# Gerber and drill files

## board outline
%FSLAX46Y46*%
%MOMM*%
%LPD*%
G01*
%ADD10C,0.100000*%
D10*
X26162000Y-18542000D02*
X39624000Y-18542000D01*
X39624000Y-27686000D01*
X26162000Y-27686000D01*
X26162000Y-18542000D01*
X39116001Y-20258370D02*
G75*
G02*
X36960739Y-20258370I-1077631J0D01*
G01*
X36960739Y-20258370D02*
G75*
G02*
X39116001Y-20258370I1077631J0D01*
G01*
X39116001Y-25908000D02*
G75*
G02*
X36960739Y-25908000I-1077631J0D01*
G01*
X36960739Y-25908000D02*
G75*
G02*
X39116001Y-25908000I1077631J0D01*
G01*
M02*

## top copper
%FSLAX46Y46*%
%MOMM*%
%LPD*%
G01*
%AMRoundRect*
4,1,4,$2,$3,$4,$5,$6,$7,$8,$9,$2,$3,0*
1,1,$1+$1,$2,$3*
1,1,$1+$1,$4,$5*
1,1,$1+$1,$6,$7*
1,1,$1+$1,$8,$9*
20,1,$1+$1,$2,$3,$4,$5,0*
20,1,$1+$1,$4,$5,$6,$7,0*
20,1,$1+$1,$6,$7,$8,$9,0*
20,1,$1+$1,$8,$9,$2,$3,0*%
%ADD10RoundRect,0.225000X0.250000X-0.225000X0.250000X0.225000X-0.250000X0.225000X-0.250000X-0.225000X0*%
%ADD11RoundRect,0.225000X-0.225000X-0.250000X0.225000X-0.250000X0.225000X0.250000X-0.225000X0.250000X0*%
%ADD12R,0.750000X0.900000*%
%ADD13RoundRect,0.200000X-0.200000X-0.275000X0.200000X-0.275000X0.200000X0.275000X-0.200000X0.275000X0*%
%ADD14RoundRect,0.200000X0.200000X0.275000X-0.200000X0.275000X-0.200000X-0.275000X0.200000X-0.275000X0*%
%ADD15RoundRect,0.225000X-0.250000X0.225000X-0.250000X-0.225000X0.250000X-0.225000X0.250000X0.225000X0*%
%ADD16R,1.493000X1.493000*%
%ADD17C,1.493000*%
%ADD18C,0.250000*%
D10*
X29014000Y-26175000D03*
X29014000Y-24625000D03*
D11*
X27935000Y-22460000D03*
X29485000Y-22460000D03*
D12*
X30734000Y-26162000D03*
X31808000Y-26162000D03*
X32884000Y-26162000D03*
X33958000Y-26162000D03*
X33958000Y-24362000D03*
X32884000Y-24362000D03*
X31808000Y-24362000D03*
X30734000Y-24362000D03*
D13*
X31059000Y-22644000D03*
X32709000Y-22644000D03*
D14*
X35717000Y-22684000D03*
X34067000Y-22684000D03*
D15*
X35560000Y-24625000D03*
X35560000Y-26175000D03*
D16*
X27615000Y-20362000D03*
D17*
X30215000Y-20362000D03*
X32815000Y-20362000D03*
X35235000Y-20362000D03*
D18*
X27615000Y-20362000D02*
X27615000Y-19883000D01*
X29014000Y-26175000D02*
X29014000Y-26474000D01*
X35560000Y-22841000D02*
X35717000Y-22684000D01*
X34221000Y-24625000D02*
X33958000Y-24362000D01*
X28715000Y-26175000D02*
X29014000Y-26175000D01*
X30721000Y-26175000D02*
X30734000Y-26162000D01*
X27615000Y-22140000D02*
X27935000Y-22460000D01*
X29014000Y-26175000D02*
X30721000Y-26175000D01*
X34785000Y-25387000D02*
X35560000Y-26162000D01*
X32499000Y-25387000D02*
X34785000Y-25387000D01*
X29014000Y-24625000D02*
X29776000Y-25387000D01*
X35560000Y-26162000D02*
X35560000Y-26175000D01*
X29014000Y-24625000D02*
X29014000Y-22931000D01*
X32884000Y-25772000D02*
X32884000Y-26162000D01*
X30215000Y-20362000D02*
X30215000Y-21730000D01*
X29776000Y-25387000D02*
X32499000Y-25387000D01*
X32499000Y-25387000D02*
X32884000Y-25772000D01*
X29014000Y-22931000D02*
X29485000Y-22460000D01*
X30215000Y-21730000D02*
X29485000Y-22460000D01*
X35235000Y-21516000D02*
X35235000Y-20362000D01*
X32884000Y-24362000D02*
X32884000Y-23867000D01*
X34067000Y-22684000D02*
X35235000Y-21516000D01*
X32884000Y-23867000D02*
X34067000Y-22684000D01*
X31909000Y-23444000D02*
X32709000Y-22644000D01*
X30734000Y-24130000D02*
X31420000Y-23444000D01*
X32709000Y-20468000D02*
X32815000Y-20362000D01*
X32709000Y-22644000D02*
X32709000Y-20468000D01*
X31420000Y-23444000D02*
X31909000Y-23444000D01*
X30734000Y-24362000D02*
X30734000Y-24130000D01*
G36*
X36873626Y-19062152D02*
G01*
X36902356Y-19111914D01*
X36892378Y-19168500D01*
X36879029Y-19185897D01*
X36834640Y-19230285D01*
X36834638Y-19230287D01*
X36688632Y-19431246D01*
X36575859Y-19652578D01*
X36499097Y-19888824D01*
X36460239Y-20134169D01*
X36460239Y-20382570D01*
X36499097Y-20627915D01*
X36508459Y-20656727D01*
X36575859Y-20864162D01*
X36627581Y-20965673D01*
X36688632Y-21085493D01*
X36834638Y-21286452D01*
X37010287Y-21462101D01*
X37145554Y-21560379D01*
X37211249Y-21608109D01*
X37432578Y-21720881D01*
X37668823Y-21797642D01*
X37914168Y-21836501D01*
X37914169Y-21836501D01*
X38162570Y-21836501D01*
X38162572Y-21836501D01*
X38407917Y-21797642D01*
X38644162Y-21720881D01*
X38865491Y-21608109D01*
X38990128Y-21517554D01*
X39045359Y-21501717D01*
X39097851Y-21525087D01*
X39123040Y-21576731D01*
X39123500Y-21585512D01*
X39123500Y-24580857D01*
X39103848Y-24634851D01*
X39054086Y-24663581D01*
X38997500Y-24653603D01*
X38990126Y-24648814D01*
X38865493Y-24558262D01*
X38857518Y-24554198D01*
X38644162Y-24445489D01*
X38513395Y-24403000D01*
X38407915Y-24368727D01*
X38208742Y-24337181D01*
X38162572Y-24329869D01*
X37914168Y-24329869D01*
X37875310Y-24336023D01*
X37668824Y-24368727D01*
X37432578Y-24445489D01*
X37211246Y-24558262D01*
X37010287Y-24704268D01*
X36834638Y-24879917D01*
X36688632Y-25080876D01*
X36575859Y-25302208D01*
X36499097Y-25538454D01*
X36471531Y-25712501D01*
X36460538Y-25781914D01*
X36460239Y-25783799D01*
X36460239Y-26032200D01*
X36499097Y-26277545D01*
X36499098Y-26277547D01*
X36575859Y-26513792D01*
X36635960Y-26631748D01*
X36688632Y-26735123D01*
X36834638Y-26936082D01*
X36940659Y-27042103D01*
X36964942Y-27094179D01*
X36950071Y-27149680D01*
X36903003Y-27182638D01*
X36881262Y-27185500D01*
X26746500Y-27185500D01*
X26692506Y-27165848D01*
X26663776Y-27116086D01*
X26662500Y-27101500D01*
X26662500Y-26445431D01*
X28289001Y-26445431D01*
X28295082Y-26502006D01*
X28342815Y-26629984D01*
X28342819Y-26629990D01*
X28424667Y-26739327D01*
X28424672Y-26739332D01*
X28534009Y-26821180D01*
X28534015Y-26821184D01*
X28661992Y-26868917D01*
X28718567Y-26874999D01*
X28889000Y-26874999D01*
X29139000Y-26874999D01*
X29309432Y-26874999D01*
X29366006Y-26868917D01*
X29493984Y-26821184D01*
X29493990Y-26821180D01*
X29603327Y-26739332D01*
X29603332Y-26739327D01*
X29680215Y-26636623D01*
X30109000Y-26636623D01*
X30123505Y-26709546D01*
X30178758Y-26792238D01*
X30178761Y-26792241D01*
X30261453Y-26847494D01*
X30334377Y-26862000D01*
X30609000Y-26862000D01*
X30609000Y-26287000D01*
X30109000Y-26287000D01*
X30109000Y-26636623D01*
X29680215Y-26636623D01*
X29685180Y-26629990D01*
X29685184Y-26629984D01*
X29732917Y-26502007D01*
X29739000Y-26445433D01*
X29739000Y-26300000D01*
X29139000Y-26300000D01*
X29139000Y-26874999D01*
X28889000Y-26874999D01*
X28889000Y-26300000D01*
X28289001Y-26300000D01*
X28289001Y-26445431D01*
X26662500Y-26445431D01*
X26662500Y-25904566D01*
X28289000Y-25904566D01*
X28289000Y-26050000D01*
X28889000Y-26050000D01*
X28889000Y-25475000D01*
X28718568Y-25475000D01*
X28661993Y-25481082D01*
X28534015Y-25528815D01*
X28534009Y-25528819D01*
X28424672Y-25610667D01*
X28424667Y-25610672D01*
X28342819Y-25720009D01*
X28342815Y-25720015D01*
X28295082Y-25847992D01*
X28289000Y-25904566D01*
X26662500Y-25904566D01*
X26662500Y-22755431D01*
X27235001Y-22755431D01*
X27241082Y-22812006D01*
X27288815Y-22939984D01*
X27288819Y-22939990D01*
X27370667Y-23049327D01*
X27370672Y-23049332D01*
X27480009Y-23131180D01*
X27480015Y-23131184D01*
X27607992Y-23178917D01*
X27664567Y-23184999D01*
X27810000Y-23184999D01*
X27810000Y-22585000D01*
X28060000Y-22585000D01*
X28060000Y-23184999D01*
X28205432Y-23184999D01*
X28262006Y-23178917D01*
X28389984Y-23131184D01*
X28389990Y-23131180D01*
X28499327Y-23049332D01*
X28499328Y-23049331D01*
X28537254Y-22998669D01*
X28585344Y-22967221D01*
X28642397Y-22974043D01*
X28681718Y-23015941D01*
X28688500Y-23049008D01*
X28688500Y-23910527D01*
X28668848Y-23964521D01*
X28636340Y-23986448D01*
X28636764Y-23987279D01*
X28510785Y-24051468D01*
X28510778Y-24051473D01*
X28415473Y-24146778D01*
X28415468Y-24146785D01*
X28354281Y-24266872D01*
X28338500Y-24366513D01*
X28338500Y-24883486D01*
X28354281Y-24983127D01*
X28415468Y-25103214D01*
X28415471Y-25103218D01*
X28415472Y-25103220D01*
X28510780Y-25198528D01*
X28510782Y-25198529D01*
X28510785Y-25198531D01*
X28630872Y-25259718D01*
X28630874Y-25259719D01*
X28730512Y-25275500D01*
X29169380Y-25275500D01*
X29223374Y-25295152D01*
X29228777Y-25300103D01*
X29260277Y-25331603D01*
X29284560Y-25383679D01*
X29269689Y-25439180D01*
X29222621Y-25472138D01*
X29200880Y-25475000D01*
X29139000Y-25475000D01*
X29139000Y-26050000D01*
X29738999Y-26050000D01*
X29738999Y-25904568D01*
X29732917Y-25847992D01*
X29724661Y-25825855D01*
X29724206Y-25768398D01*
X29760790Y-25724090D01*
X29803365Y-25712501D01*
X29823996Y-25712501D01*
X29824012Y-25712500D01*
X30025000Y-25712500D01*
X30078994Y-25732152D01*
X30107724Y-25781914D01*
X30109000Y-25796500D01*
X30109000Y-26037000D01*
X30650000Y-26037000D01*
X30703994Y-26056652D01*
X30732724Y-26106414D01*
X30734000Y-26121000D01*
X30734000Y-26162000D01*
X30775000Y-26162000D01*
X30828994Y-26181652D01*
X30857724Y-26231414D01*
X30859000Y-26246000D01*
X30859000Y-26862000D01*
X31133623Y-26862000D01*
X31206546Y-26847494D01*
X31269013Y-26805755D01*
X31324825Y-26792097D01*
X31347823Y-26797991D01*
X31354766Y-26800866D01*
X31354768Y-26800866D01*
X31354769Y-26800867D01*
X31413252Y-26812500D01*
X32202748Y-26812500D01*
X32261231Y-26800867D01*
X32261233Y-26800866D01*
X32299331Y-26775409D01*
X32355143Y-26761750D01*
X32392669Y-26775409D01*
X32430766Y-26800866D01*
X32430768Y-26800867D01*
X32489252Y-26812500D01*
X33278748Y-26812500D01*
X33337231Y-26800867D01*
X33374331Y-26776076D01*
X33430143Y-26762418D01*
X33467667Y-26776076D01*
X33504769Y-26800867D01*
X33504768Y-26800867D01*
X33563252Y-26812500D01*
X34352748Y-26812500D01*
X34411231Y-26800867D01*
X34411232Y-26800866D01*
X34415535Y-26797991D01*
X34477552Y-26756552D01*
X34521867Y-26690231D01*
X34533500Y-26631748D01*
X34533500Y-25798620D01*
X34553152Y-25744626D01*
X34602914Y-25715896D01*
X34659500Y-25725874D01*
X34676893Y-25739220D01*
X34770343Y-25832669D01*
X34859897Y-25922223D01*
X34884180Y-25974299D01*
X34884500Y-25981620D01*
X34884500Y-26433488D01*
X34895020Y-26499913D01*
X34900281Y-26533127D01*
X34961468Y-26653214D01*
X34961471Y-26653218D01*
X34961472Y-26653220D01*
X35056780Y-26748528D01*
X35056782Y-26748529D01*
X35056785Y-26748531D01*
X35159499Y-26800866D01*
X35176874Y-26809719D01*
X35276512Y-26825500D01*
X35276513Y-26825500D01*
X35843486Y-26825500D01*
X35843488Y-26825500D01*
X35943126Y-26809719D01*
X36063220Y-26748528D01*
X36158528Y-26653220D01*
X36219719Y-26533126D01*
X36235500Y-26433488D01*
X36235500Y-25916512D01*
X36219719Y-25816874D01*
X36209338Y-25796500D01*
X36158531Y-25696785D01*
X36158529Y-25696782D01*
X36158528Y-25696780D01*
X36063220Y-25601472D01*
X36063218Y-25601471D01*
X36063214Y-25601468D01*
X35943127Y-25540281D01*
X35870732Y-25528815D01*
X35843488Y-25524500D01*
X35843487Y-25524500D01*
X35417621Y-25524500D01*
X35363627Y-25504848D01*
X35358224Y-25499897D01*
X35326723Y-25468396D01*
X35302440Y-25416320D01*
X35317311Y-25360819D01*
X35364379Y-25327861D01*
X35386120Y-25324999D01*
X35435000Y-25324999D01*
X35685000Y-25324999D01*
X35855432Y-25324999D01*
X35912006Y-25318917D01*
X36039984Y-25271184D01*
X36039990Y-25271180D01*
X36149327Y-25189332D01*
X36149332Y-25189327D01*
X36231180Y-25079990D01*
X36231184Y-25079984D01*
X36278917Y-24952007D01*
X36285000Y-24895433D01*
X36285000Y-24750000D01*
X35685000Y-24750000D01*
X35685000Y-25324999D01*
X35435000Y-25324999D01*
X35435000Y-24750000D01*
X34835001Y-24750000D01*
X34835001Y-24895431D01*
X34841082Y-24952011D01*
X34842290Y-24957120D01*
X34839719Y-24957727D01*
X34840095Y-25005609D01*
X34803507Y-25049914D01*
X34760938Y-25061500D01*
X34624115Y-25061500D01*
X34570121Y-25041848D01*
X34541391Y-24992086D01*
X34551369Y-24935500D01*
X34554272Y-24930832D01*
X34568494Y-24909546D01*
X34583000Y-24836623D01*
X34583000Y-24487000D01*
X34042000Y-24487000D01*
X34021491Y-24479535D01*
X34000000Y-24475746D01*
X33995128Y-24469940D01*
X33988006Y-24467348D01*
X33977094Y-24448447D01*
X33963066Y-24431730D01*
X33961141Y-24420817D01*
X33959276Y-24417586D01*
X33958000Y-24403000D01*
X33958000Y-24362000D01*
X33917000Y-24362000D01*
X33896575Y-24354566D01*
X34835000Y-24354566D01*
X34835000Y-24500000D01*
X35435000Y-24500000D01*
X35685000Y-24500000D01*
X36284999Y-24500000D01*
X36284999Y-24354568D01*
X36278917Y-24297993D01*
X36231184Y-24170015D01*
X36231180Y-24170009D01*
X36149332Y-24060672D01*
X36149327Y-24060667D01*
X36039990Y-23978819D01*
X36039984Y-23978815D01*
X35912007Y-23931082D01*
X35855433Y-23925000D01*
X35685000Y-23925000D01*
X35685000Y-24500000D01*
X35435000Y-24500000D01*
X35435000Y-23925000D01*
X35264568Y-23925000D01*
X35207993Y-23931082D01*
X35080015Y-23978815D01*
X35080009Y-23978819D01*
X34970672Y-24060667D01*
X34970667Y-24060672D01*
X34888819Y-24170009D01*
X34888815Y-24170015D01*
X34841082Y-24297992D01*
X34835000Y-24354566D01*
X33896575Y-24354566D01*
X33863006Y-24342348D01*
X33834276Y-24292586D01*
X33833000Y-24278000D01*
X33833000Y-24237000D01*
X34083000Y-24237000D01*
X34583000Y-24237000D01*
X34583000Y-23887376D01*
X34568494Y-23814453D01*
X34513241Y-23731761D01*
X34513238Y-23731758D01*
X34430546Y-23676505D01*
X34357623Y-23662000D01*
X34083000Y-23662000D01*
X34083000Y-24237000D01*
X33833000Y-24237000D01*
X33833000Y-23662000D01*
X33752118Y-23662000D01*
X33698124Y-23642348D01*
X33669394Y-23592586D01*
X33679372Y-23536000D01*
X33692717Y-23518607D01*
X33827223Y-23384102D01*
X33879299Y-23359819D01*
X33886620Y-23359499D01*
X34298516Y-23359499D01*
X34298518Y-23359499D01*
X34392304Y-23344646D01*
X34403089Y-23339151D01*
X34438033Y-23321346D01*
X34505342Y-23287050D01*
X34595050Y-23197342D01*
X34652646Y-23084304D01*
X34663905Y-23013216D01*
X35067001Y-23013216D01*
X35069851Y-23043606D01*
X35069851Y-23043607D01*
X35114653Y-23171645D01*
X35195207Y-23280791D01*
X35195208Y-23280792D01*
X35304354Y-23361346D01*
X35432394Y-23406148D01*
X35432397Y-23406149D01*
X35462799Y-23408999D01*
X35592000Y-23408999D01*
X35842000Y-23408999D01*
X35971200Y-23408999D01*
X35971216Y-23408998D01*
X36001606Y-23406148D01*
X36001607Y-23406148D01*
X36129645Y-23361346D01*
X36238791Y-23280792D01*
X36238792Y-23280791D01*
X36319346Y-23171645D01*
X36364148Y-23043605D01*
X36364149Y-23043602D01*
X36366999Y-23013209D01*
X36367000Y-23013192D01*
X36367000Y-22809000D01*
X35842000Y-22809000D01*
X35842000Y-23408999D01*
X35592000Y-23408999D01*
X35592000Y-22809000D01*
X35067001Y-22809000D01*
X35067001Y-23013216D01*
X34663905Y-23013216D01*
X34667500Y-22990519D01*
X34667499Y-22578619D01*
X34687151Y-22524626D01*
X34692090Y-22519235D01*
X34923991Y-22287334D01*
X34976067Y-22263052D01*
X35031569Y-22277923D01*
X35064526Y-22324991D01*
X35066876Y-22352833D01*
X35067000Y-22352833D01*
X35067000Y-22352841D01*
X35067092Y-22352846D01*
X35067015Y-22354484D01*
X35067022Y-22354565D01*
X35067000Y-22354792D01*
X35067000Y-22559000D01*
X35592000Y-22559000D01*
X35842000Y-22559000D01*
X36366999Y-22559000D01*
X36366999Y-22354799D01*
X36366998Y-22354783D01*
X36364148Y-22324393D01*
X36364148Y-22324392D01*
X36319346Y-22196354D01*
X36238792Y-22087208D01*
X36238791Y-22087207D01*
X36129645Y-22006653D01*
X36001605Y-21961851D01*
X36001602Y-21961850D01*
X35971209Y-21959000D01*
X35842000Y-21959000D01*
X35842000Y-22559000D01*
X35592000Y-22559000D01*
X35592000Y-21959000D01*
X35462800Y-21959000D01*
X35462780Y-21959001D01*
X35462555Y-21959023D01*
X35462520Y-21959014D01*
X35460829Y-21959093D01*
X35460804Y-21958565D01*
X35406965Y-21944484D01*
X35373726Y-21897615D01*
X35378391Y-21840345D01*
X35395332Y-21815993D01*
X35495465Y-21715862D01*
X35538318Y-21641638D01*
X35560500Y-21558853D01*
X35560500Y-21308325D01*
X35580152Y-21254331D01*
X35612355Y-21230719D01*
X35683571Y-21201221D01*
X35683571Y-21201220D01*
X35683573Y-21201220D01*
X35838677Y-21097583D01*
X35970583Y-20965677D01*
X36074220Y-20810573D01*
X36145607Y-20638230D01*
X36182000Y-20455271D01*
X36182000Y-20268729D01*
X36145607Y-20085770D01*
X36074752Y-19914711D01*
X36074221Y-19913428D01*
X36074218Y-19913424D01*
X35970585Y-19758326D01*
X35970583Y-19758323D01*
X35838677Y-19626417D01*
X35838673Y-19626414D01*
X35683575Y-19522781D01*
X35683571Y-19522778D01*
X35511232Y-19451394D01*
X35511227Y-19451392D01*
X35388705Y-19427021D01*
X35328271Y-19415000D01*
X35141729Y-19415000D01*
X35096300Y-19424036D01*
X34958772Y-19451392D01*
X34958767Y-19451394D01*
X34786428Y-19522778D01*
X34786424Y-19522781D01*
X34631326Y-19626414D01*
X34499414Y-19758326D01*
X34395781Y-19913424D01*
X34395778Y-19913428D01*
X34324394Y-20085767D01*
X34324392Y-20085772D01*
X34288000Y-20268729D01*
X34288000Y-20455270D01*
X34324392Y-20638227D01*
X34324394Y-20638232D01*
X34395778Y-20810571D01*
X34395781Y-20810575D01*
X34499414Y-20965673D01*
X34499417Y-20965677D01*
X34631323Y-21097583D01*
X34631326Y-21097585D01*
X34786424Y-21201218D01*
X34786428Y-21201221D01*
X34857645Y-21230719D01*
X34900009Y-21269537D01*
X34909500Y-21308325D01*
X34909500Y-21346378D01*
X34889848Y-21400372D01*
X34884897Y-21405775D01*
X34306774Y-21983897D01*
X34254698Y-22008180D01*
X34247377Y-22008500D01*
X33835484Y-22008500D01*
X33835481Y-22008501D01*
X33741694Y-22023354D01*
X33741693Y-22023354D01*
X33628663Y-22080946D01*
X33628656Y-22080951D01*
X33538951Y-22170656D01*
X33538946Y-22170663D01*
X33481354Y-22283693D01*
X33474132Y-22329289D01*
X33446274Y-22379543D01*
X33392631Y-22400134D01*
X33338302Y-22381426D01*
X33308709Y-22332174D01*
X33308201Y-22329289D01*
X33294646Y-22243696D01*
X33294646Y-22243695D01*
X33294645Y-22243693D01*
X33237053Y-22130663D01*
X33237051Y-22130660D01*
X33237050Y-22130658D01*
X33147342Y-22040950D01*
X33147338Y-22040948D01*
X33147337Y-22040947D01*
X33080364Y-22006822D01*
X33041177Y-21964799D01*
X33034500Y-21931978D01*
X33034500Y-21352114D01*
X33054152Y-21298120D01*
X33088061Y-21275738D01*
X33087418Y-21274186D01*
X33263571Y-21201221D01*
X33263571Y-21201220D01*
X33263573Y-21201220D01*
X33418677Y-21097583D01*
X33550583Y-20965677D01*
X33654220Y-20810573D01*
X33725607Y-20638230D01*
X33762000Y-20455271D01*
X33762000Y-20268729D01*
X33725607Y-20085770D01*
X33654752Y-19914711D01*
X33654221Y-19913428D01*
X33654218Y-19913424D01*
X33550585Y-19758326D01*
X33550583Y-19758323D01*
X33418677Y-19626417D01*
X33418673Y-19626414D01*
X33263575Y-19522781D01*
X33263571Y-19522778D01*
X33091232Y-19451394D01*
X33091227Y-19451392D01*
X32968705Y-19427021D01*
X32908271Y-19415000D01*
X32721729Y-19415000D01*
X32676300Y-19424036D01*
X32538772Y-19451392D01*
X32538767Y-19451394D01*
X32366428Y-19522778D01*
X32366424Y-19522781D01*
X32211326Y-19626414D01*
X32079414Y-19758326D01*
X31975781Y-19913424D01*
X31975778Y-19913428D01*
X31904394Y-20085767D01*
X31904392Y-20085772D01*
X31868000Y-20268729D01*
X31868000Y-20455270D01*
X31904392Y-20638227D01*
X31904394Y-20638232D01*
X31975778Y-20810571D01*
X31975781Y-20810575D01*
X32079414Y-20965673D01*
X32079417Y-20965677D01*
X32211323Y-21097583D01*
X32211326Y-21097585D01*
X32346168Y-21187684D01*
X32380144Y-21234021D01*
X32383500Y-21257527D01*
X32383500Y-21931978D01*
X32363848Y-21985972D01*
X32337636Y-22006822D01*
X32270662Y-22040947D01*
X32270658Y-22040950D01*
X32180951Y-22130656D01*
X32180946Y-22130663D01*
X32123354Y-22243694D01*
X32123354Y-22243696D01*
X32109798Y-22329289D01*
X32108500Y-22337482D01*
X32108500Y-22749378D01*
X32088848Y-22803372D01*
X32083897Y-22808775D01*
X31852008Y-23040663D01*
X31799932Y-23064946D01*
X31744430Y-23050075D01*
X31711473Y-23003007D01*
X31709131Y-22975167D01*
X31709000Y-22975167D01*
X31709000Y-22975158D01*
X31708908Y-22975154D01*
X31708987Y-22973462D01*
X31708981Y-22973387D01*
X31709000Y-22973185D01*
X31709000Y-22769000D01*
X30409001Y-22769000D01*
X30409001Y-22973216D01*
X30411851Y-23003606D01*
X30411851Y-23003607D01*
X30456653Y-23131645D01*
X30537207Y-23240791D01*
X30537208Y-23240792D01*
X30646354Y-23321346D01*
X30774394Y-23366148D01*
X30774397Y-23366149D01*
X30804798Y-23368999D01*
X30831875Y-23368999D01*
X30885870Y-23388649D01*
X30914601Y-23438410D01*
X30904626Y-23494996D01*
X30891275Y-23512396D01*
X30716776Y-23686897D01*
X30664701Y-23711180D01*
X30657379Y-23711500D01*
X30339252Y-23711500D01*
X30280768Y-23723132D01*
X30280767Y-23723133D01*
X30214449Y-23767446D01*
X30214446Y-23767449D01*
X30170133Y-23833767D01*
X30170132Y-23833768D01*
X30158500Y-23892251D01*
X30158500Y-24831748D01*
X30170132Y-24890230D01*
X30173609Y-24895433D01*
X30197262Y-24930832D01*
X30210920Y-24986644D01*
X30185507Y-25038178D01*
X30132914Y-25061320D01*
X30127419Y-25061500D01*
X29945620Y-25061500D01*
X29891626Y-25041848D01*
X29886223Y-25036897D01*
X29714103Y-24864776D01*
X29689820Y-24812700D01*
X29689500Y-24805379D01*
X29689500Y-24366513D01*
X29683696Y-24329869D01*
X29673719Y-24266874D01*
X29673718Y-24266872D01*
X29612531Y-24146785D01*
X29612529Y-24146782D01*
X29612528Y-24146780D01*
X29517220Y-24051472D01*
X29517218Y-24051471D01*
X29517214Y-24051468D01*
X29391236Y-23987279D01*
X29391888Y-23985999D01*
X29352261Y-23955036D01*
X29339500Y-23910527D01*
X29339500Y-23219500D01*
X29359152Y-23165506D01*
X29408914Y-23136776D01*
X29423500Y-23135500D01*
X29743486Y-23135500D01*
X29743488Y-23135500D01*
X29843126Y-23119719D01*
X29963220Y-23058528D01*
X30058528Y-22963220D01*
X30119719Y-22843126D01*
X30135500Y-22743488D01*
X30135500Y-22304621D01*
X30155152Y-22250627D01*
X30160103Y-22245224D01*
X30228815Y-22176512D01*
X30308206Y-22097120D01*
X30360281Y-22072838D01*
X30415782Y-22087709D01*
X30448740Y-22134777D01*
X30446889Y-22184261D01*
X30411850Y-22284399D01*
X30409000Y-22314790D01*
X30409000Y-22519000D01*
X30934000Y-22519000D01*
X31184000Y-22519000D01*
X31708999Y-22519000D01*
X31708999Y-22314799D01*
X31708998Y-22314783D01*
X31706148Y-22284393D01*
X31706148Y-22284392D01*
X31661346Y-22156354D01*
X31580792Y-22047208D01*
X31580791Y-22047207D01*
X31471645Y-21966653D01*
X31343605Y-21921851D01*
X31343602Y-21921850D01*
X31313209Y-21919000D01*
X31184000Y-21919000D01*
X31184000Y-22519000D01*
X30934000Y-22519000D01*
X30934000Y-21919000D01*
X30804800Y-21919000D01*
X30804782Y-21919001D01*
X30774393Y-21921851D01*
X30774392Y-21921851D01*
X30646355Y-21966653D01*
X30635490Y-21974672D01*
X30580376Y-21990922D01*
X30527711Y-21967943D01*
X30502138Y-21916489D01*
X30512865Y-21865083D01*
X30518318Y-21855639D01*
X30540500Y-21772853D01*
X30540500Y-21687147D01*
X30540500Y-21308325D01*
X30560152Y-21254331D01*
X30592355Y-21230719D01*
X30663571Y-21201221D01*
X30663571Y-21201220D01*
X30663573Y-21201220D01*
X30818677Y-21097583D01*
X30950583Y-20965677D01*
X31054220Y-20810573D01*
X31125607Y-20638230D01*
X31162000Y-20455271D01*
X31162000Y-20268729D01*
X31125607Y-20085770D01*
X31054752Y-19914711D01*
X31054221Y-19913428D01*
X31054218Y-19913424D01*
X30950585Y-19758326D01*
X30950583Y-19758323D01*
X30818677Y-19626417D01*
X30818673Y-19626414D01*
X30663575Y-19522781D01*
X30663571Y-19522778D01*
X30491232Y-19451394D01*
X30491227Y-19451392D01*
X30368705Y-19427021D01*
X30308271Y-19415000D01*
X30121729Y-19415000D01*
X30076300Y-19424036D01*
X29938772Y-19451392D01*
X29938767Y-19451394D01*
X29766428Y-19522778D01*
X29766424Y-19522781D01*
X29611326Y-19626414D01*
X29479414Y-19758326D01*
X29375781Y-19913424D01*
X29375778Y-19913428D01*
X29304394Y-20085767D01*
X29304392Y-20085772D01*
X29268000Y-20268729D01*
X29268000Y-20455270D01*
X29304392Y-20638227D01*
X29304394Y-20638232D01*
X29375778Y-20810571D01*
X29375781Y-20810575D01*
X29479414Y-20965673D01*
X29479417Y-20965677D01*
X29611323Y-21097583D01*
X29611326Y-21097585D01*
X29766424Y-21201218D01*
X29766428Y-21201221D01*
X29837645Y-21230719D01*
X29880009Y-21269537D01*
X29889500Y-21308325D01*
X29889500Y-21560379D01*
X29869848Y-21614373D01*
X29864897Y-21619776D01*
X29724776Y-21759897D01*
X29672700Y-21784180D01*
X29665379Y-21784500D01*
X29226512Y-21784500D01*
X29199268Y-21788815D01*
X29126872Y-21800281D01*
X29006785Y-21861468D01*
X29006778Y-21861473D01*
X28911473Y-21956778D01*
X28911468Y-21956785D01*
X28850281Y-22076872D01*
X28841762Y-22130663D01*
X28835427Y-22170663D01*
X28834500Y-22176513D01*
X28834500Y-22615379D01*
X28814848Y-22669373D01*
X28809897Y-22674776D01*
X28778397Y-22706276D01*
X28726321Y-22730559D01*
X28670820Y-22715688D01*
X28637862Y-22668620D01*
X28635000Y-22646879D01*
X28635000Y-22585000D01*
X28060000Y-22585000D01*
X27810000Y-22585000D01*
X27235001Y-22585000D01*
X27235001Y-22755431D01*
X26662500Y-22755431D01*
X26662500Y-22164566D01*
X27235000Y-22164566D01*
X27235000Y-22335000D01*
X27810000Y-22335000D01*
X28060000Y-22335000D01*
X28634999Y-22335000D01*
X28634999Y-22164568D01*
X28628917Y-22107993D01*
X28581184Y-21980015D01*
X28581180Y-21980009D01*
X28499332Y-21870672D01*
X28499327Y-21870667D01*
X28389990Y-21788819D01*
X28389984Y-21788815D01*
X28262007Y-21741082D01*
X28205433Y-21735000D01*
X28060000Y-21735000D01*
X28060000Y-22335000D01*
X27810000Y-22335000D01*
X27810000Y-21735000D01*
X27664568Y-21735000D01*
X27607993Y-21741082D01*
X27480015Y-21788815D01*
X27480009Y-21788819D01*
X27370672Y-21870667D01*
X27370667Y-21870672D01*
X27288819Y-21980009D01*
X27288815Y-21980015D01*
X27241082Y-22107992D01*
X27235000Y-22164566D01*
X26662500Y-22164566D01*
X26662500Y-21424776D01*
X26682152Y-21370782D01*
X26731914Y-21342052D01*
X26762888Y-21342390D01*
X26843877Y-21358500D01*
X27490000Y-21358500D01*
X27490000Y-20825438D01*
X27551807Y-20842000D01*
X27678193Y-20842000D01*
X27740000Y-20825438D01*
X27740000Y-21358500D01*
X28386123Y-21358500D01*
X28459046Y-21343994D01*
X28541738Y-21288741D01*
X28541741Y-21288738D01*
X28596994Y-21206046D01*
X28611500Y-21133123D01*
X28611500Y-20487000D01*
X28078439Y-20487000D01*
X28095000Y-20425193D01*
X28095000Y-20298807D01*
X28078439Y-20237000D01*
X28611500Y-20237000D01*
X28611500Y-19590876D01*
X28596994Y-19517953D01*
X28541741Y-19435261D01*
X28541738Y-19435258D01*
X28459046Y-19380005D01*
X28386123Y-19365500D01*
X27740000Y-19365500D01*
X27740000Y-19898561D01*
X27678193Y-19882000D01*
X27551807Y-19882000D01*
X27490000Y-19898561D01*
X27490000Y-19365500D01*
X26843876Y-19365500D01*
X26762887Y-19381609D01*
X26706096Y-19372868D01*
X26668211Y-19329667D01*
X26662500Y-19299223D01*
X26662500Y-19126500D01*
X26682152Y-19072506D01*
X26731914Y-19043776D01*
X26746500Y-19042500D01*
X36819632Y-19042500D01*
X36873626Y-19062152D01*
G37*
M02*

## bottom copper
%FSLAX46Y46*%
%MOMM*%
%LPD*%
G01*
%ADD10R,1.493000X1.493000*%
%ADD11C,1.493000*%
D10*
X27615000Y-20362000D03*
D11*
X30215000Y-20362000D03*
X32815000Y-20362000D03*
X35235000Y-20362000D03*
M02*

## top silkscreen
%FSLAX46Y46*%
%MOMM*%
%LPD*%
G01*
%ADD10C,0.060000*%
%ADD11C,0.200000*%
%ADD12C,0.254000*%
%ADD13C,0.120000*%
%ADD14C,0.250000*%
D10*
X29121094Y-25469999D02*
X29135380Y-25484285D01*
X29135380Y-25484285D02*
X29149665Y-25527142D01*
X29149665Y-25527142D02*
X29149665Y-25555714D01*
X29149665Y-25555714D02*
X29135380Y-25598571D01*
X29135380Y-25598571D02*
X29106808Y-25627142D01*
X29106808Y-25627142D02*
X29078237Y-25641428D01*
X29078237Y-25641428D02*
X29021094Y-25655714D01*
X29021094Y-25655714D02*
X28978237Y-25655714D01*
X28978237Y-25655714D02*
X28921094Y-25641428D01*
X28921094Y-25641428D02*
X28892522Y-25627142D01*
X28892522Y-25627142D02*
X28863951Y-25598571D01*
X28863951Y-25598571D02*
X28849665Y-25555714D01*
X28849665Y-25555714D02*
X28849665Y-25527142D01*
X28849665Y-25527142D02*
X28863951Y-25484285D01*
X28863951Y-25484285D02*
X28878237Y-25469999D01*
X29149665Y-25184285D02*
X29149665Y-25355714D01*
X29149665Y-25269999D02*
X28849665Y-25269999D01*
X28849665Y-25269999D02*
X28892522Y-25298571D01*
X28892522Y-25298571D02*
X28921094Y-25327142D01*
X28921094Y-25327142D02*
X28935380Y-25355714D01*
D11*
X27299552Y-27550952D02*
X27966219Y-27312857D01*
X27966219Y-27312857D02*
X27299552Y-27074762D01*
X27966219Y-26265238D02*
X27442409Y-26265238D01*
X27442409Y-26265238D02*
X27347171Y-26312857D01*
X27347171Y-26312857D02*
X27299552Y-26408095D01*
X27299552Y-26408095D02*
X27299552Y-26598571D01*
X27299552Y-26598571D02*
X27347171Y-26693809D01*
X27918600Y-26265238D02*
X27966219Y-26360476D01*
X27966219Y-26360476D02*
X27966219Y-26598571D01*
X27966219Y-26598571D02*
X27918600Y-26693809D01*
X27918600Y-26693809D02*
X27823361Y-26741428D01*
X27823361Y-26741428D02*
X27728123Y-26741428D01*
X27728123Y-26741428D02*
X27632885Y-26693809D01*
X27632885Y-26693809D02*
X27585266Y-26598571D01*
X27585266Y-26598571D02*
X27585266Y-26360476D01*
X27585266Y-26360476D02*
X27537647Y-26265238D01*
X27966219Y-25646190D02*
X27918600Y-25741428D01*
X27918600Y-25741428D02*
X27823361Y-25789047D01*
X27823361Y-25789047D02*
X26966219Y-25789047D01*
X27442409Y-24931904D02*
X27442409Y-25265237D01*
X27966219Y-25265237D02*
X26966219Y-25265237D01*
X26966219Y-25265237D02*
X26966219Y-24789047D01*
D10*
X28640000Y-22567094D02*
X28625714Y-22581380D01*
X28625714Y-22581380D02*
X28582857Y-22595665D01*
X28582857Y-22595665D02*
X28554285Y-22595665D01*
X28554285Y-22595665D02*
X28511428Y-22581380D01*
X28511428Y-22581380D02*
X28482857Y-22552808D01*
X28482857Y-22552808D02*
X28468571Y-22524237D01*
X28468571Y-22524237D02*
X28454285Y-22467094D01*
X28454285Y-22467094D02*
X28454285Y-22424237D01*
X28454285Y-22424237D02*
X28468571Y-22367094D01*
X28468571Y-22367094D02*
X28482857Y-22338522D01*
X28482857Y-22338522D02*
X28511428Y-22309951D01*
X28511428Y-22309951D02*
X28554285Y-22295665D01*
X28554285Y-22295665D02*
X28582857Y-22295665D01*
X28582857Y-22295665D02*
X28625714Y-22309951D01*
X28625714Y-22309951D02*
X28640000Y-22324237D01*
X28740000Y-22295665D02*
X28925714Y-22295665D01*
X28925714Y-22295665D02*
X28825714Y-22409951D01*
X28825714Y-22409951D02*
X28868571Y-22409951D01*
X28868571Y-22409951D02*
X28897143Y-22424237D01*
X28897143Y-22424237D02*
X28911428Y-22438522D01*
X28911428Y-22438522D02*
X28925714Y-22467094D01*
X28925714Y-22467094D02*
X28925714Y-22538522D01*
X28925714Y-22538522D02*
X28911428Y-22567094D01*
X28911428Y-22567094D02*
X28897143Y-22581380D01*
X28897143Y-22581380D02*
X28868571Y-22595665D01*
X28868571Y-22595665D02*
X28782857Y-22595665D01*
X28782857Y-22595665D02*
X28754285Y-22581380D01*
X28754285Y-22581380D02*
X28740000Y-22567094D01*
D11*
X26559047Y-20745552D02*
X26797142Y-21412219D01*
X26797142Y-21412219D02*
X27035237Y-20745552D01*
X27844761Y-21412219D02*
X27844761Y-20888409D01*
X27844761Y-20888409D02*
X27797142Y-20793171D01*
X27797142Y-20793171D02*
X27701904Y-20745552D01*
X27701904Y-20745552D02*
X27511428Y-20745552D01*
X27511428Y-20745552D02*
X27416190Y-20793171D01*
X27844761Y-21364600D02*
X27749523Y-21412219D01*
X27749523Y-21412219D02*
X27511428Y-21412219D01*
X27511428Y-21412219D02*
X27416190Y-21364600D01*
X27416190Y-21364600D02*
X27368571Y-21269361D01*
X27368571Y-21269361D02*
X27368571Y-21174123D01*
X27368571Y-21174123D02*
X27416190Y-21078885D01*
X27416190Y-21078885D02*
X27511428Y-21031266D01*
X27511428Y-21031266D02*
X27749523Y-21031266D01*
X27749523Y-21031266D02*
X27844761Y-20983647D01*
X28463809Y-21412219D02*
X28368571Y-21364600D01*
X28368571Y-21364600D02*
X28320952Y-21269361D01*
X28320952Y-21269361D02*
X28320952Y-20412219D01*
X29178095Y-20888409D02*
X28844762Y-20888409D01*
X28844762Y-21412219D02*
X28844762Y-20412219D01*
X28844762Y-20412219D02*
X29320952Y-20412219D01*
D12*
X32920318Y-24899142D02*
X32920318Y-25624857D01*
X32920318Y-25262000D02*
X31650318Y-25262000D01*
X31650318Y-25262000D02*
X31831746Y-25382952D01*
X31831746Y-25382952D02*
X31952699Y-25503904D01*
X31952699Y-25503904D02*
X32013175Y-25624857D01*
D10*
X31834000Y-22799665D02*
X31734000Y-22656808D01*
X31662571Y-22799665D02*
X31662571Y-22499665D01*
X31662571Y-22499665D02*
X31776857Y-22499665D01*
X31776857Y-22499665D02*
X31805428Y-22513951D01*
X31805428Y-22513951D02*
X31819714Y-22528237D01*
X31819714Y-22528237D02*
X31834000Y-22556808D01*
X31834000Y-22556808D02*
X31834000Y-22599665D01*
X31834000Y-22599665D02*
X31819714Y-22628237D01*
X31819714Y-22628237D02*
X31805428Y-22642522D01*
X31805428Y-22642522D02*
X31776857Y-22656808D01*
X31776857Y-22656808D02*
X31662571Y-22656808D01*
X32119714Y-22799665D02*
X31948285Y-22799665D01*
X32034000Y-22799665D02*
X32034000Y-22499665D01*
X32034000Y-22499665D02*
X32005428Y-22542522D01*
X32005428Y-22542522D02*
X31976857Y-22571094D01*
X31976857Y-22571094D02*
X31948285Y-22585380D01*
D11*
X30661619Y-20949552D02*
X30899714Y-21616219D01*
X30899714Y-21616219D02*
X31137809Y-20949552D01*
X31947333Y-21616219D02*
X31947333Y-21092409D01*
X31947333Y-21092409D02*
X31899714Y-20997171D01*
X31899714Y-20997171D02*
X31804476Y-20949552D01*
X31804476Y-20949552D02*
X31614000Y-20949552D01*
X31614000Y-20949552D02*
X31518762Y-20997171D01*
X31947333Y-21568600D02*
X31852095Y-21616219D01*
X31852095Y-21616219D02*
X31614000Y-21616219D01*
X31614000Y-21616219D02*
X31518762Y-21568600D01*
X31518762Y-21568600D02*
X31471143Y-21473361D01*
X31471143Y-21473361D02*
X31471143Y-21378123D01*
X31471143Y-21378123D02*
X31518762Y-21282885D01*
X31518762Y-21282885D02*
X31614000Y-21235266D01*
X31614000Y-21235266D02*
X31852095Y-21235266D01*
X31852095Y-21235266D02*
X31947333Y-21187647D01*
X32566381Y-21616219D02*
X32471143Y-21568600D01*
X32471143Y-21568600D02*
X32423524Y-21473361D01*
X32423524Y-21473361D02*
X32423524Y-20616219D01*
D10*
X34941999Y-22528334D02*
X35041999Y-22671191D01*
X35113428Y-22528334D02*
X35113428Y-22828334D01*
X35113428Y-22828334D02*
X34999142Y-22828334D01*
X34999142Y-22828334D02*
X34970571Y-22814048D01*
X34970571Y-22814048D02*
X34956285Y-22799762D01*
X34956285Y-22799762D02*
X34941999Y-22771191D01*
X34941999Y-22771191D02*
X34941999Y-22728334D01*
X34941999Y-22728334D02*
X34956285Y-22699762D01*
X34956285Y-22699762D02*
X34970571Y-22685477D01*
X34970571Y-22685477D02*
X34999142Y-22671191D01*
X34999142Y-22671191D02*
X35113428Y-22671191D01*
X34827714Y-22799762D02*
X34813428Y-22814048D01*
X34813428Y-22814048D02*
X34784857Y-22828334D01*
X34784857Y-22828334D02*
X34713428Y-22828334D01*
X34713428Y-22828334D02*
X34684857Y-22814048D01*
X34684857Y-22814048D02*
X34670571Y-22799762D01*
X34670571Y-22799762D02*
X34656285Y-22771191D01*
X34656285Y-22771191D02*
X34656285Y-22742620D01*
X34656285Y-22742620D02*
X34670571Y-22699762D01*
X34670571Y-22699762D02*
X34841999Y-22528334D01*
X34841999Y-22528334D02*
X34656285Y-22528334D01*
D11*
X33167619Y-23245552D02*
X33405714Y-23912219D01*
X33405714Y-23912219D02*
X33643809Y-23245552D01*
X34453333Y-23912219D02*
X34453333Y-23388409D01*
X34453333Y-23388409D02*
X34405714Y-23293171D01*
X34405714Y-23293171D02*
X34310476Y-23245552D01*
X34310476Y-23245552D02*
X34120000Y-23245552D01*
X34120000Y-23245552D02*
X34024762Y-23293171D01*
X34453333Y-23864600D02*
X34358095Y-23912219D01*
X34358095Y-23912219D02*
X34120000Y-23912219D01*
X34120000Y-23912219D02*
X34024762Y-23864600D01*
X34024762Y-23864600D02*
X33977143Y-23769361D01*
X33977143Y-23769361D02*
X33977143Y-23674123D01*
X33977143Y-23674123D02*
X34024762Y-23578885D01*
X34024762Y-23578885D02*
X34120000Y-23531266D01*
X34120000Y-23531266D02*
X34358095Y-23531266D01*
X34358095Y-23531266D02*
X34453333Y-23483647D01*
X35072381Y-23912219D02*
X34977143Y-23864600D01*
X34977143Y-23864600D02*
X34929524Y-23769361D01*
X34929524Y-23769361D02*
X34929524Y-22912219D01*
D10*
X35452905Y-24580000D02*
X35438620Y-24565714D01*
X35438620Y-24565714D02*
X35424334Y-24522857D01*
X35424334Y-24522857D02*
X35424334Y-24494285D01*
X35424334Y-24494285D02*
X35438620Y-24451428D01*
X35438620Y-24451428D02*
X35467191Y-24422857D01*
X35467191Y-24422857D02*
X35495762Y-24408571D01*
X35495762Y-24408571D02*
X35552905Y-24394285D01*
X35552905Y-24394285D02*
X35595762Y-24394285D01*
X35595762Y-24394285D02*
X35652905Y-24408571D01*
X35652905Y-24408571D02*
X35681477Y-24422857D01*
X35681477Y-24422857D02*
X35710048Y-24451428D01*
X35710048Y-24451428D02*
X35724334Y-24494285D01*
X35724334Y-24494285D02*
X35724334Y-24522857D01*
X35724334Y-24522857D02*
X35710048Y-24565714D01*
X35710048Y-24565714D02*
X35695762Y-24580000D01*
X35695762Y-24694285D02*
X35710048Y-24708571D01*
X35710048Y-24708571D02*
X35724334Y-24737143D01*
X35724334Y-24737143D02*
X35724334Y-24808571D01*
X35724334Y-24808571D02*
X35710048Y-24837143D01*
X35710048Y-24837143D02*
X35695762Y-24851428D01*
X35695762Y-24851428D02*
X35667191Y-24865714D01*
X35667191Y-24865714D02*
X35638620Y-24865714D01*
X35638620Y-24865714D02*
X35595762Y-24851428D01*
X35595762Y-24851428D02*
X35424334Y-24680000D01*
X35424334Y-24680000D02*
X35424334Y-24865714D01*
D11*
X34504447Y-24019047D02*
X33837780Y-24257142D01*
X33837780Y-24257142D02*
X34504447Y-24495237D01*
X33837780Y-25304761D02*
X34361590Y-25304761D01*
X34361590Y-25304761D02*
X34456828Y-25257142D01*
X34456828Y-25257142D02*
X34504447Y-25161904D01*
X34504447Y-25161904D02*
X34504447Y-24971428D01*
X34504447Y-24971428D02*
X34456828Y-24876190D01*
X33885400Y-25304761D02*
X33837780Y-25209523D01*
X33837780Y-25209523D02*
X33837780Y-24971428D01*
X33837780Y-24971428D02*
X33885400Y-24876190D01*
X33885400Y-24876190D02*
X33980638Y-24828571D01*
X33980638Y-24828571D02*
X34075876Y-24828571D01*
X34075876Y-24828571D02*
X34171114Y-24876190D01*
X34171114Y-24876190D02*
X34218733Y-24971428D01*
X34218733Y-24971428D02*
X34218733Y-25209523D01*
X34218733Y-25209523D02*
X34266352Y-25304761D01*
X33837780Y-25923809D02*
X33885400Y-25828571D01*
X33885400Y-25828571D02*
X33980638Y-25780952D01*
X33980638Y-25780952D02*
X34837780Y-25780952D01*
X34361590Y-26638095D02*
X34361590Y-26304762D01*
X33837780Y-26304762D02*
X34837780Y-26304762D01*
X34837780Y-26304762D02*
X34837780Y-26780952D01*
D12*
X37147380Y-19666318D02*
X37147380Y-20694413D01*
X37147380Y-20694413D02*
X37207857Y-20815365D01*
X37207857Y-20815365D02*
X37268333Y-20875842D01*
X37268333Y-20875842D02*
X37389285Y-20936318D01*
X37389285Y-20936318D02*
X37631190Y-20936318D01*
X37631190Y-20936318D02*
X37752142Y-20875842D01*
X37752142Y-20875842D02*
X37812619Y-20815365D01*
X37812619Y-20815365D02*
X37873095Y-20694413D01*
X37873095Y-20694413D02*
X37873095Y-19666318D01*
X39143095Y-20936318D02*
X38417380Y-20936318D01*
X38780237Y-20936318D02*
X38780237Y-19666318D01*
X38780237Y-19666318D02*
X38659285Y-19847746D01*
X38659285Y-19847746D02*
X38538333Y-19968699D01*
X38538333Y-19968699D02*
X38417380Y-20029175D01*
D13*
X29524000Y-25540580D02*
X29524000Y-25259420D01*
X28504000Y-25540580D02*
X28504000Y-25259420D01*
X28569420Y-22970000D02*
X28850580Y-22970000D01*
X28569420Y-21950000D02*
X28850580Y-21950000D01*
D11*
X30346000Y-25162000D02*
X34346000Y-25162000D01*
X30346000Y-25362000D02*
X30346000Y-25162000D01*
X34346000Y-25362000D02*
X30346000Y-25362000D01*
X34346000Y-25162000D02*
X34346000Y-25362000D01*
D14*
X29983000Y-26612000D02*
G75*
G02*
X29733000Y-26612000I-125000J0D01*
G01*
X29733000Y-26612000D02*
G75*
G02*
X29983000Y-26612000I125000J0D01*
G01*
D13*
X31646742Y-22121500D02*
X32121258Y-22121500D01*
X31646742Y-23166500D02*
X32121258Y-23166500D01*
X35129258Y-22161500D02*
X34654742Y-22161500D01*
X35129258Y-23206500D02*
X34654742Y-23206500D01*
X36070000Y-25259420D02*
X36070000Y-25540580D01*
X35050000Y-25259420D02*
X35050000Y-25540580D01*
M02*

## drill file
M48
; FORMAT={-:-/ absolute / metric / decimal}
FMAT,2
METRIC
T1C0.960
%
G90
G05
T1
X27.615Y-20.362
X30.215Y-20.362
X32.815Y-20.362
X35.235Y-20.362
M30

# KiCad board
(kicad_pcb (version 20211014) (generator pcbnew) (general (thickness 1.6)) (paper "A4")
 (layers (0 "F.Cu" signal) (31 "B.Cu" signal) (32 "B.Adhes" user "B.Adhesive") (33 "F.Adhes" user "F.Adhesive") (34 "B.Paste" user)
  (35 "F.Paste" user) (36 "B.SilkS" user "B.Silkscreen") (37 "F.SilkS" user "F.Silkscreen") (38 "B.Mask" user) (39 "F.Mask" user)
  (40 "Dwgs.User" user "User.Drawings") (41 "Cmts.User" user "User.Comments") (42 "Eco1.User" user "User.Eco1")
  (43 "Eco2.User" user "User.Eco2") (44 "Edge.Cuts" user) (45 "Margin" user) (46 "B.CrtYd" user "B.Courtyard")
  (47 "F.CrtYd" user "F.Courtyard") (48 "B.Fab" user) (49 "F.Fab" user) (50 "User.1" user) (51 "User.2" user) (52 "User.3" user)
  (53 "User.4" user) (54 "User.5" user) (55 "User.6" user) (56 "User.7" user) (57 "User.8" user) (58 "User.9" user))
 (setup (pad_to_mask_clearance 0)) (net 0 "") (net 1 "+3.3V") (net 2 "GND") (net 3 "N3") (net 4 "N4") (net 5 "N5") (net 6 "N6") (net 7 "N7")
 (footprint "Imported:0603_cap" (layer "F.Cu") (at 29.014 26.17 90)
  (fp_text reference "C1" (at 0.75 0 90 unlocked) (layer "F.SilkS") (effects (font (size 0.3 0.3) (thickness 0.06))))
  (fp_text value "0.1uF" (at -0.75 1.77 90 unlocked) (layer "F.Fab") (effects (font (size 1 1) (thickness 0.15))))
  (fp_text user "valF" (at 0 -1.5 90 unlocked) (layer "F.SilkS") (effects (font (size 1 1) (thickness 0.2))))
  (fp_line (start 0.62942 0.51) (end 0.91058 0.51) (layer "F.SilkS") (width 0.12))
  (fp_line (start 0.62942 -0.51) (end 0.91058 -0.51) (layer "F.SilkS") (width 0.12))
  (pad "1" smd roundrect (at -0.005 0 90) (size 0.9 0.95) (layers "F.Cu" "F.Paste" "F.Mask") (roundrect_rratio 0.25) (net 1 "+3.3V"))
  (pad "2" smd roundrect (at 1.545 0 90) (size 0.9 0.95) (layers "F.Cu" "F.Paste" "F.Mask") (roundrect_rratio 0.25) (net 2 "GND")))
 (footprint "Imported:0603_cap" (layer "F.Cu") (at 27.94 22.46)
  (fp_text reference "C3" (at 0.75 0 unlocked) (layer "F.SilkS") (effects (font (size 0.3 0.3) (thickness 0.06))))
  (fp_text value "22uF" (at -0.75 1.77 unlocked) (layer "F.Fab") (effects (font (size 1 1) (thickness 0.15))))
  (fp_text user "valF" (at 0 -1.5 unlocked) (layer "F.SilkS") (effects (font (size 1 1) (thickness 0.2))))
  (fp_line (start 0.62942 0.51) (end 0.91058 0.51) (layer "F.SilkS") (width 0.12))
  (fp_line (start 0.62942 -0.51) (end 0.91058 -0.51) (layer "F.SilkS") (width 0.12))
  (pad "1" smd roundrect (at -0.005 0) (size 0.9 0.95) (layers "F.Cu" "F.Paste" "F.Mask") (roundrect_rratio 0.25) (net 1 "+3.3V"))
  (pad "2" smd roundrect (at 1.545 0) (size 0.9 0.95) (layers "F.Cu" "F.Paste" "F.Mask") (roundrect_rratio 0.25) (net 2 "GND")))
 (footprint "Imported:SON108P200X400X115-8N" (layer "F.Cu") (at 32.346 25.262 90)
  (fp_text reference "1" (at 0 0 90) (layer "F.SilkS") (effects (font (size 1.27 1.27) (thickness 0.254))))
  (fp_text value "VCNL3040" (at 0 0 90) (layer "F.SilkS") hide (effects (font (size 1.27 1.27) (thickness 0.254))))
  (fp_line (start 0.1 -2) (end 0.1 2) (layer "F.SilkS") (width 0.2))
  (fp_line (start -0.1 -2) (end 0.1 -2) (layer "F.SilkS") (width 0.2))
  (fp_line (start -0.1 2) (end -0.1 -2) (layer "F.SilkS") (width 0.2))
  (fp_line (start 0.1 2) (end -0.1 2) (layer "F.SilkS") (width 0.2))
  (fp_circle (center -1.35 -2.488) (end -1.35 -2.363) (layer "F.SilkS") (width 0.25) (fill none))
  (pad "1" smd rect (at -0.9 -1.612 180) (size 0.75 0.9) (layers "F.Cu" "F.Paste" "F.Mask") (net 1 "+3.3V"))
  (pad "2" smd rect (at -0.9 -0.538 180) (size 0.75 0.9) (layers "F.Cu" "F.Paste" "F.Mask") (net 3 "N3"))
  (pad "3" smd rect (at -0.9 0.538 180) (size 0.75 0.9) (layers "F.Cu" "F.Paste" "F.Mask") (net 2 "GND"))
  (pad "4" smd rect (at -0.9 1.612 180) (size 0.75 0.9) (layers "F.Cu" "F.Paste" "F.Mask") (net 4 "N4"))
  (pad "5" smd rect (at 0.9 1.612 180) (size 0.75 0.9) (layers "F.Cu" "F.Paste" "F.Mask") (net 1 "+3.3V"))
  (pad "6" smd rect (at 0.9 0.538 180) (size 0.75 0.9) (layers "F.Cu" "F.Paste" "F.Mask") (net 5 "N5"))
  (pad "7" smd rect (at 0.9 -0.538 180) (size 0.75 0.9) (layers "F.Cu" "F.Paste" "F.Mask") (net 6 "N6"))
  (pad "8" smd rect (at 0.9 -1.612 180) (size 0.75 0.9) (layers "F.Cu" "F.Paste" "F.Mask") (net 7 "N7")))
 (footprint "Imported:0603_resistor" (layer "F.Cu") (at 31.864 22.664)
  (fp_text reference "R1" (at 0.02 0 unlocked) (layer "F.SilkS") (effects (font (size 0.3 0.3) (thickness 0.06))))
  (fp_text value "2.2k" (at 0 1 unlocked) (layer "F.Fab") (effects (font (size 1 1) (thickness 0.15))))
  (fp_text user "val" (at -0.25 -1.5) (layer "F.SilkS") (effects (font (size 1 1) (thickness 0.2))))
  (fp_line (start -0.217258 -0.5425) (end 0.257258 -0.5425) (layer "F.SilkS") (width 0.12))
  (fp_line (start -0.217258 0.5025) (end 0.257258 0.5025) (layer "F.SilkS") (width 0.12))
  (pad "1" smd roundrect (at -0.805 -0.02) (size 0.8 0.95) (layers "F.Cu" "F.Paste" "F.Mask") (roundrect_rratio 0.25) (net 1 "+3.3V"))
  (pad "2" smd roundrect (at 0.845 -0.02) (size 0.8 0.95) (layers "F.Cu" "F.Paste" "F.Mask") (roundrect_rratio 0.25) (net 7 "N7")))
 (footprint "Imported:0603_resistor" (layer "F.Cu") (at 34.912 22.664 180)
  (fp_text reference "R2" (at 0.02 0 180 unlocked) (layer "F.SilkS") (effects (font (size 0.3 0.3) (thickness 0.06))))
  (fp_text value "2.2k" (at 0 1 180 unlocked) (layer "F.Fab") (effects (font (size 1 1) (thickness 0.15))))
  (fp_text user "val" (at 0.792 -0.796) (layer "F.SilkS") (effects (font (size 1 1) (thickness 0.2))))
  (fp_line (start -0.217258 0.5025) (end 0.257258 0.5025) (layer "F.SilkS") (width 0.12))
  (fp_line (start -0.217258 -0.5425) (end 0.257258 -0.5425) (layer "F.SilkS") (width 0.12))
  (pad "1" smd roundrect (at -0.805 -0.02 180) (size 0.8 0.95) (layers "F.Cu" "F.Paste" "F.Mask") (roundrect_rratio 0.25) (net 1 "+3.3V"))
  (pad "2" smd roundrect (at 0.845 -0.02 180) (size 0.8 0.95) (layers "F.Cu" "F.Paste" "F.Mask") (roundrect_rratio 0.25) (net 5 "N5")))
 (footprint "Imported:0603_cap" (layer "F.Cu") (at 35.56 24.63 -90)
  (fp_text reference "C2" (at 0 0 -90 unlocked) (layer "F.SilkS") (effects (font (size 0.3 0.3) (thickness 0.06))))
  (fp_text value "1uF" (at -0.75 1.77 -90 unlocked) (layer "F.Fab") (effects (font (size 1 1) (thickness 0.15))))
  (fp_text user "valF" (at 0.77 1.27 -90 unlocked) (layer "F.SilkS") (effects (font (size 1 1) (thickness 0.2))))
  (fp_line (start 0.62942 -0.51) (end 0.91058 -0.51) (layer "F.SilkS") (width 0.12))
  (fp_line (start 0.62942 0.51) (end 0.91058 0.51) (layer "F.SilkS") (width 0.12))
  (pad "1" smd roundrect (at -0.005 0 270) (size 0.9 0.95) (layers "F.Cu" "F.Paste" "F.Mask") (roundrect_rratio 0.25) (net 1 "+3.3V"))
  (pad "2" smd roundrect (at 1.545 0 270) (size 0.9 0.95) (layers "F.Cu" "F.Paste" "F.Mask") (roundrect_rratio 0.25) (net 2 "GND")))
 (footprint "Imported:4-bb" (layer "F.Cu") (at 27.615 20.362)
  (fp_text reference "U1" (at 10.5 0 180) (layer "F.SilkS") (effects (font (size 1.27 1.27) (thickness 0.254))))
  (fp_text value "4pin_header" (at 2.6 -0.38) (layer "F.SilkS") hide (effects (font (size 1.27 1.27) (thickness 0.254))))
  (pad "1" thru_hole rect (at 0 0) (size 1.493 1.493) (drill 0.96) (layers *.Cu *.Mask) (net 1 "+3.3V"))
  (pad "2" thru_hole circle (at 2.6 0) (size 1.493 1.493) (drill 0.96) (layers *.Cu *.Mask) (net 2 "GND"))
  (pad "3" thru_hole circle (at 5.2 0) (size 1.493 1.493) (drill 0.96) (layers *.Cu *.Mask) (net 7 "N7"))
  (pad "4" thru_hole circle (at 7.62 0) (size 1.493 1.493) (drill 0.96) (layers *.Cu *.Mask) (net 5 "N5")))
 (gr_rect (start 39.624 18.542) (end 26.162 27.686) (layer "Edge.Cuts") (width 0.1) (fill none))
 (gr_circle (center 38.03837 20.25837) (end 37.27637 19.49637) (layer "Edge.Cuts") (width 0.1) (fill none))
 (gr_circle (center 38.03837 25.908) (end 37.27637 25.146) (layer "Edge.Cuts") (width 0.1) (fill none))
 (segment (start 27.615 20.362) (end 27.615 19.883) (width 0.25) (layer "F.Cu") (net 1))
 (segment (start 29.014 26.175) (end 29.014 26.474) (width 0.25) (layer "F.Cu") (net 1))
 (segment (start 35.56 22.841) (end 35.717 22.684) (width 0.25) (layer "F.Cu") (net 1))
 (segment (start 34.221 24.625) (end 33.958 24.362) (width 0.25) (layer "F.Cu") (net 1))
 (segment (start 28.715 26.175) (end 29.014 26.175) (width 0.25) (layer "F.Cu") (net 1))
 (segment (start 30.721 26.175) (end 30.734 26.162) (width 0.25) (layer "F.Cu") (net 1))
 (segment (start 27.615 22.14) (end 27.935 22.46) (width 0.25) (layer "F.Cu") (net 1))
 (segment (start 29.014 26.175) (end 30.721 26.175) (width 0.25) (layer "F.Cu") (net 1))
 (segment (start 34.785 25.387) (end 35.56 26.162) (width 0.25) (layer "F.Cu") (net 2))
 (segment (start 32.499 25.387) (end 34.785 25.387) (width 0.25) (layer "F.Cu") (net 2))
 (segment (start 29.014 24.625) (end 29.776 25.387) (width 0.25) (layer "F.Cu") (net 2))
 (segment (start 35.56 26.162) (end 35.56 26.175) (width 0.25) (layer "F.Cu") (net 2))
 (segment (start 29.014 24.625) (end 29.014 22.931) (width 0.25) (layer "F.Cu") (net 2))
 (segment (start 32.884 25.772) (end 32.884 26.162) (width 0.25) (layer "F.Cu") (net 2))
 (segment (start 30.215 20.362) (end 30.215 21.73) (width 0.25) (layer "F.Cu") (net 2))
 (segment (start 29.776 25.387) (end 32.499 25.387) (width 0.25) (layer "F.Cu") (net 2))
 (segment (start 32.499 25.387) (end 32.884 25.772) (width 0.25) (layer "F.Cu") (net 2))
 (segment (start 29.014 22.931) (end 29.485 22.46) (width 0.25) (layer "F.Cu") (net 2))
 (segment (start 30.215 21.73) (end 29.485 22.46) (width 0.25) (layer "F.Cu") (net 2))
 (segment (start 35.235 21.516) (end 35.235 20.362) (width 0.25) (layer "F.Cu") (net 5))
 (segment (start 32.884 24.362) (end 32.884 23.867) (width 0.25) (layer "F.Cu") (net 5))
 (segment (start 34.067 22.684) (end 35.235 21.516) (width 0.25) (layer "F.Cu") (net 5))
 (segment (start 32.884 23.867) (end 34.067 22.684) (width 0.25) (layer "F.Cu") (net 5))
 (segment (start 31.909 23.444) (end 32.709 22.644) (width 0.25) (layer "F.Cu") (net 7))
 (segment (start 30.734 24.13) (end 31.42 23.444) (width 0.25) (layer "F.Cu") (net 7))
 (segment (start 32.709 20.468) (end 32.815 20.362) (width 0.25) (layer "F.Cu") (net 7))
 (segment (start 32.709 22.644) (end 32.709 20.468) (width 0.25) (layer "F.Cu") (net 7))
 (segment (start 31.42 23.444) (end 31.909 23.444) (width 0.25) (layer "F.Cu") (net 7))
 (segment (start 30.734 24.362) (end 30.734 24.13) (width 0.25) (layer "F.Cu") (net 7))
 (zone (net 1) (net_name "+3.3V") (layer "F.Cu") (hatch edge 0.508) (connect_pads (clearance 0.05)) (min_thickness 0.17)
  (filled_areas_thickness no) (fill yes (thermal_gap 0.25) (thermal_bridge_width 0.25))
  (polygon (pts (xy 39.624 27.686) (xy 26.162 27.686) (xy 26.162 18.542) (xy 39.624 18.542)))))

